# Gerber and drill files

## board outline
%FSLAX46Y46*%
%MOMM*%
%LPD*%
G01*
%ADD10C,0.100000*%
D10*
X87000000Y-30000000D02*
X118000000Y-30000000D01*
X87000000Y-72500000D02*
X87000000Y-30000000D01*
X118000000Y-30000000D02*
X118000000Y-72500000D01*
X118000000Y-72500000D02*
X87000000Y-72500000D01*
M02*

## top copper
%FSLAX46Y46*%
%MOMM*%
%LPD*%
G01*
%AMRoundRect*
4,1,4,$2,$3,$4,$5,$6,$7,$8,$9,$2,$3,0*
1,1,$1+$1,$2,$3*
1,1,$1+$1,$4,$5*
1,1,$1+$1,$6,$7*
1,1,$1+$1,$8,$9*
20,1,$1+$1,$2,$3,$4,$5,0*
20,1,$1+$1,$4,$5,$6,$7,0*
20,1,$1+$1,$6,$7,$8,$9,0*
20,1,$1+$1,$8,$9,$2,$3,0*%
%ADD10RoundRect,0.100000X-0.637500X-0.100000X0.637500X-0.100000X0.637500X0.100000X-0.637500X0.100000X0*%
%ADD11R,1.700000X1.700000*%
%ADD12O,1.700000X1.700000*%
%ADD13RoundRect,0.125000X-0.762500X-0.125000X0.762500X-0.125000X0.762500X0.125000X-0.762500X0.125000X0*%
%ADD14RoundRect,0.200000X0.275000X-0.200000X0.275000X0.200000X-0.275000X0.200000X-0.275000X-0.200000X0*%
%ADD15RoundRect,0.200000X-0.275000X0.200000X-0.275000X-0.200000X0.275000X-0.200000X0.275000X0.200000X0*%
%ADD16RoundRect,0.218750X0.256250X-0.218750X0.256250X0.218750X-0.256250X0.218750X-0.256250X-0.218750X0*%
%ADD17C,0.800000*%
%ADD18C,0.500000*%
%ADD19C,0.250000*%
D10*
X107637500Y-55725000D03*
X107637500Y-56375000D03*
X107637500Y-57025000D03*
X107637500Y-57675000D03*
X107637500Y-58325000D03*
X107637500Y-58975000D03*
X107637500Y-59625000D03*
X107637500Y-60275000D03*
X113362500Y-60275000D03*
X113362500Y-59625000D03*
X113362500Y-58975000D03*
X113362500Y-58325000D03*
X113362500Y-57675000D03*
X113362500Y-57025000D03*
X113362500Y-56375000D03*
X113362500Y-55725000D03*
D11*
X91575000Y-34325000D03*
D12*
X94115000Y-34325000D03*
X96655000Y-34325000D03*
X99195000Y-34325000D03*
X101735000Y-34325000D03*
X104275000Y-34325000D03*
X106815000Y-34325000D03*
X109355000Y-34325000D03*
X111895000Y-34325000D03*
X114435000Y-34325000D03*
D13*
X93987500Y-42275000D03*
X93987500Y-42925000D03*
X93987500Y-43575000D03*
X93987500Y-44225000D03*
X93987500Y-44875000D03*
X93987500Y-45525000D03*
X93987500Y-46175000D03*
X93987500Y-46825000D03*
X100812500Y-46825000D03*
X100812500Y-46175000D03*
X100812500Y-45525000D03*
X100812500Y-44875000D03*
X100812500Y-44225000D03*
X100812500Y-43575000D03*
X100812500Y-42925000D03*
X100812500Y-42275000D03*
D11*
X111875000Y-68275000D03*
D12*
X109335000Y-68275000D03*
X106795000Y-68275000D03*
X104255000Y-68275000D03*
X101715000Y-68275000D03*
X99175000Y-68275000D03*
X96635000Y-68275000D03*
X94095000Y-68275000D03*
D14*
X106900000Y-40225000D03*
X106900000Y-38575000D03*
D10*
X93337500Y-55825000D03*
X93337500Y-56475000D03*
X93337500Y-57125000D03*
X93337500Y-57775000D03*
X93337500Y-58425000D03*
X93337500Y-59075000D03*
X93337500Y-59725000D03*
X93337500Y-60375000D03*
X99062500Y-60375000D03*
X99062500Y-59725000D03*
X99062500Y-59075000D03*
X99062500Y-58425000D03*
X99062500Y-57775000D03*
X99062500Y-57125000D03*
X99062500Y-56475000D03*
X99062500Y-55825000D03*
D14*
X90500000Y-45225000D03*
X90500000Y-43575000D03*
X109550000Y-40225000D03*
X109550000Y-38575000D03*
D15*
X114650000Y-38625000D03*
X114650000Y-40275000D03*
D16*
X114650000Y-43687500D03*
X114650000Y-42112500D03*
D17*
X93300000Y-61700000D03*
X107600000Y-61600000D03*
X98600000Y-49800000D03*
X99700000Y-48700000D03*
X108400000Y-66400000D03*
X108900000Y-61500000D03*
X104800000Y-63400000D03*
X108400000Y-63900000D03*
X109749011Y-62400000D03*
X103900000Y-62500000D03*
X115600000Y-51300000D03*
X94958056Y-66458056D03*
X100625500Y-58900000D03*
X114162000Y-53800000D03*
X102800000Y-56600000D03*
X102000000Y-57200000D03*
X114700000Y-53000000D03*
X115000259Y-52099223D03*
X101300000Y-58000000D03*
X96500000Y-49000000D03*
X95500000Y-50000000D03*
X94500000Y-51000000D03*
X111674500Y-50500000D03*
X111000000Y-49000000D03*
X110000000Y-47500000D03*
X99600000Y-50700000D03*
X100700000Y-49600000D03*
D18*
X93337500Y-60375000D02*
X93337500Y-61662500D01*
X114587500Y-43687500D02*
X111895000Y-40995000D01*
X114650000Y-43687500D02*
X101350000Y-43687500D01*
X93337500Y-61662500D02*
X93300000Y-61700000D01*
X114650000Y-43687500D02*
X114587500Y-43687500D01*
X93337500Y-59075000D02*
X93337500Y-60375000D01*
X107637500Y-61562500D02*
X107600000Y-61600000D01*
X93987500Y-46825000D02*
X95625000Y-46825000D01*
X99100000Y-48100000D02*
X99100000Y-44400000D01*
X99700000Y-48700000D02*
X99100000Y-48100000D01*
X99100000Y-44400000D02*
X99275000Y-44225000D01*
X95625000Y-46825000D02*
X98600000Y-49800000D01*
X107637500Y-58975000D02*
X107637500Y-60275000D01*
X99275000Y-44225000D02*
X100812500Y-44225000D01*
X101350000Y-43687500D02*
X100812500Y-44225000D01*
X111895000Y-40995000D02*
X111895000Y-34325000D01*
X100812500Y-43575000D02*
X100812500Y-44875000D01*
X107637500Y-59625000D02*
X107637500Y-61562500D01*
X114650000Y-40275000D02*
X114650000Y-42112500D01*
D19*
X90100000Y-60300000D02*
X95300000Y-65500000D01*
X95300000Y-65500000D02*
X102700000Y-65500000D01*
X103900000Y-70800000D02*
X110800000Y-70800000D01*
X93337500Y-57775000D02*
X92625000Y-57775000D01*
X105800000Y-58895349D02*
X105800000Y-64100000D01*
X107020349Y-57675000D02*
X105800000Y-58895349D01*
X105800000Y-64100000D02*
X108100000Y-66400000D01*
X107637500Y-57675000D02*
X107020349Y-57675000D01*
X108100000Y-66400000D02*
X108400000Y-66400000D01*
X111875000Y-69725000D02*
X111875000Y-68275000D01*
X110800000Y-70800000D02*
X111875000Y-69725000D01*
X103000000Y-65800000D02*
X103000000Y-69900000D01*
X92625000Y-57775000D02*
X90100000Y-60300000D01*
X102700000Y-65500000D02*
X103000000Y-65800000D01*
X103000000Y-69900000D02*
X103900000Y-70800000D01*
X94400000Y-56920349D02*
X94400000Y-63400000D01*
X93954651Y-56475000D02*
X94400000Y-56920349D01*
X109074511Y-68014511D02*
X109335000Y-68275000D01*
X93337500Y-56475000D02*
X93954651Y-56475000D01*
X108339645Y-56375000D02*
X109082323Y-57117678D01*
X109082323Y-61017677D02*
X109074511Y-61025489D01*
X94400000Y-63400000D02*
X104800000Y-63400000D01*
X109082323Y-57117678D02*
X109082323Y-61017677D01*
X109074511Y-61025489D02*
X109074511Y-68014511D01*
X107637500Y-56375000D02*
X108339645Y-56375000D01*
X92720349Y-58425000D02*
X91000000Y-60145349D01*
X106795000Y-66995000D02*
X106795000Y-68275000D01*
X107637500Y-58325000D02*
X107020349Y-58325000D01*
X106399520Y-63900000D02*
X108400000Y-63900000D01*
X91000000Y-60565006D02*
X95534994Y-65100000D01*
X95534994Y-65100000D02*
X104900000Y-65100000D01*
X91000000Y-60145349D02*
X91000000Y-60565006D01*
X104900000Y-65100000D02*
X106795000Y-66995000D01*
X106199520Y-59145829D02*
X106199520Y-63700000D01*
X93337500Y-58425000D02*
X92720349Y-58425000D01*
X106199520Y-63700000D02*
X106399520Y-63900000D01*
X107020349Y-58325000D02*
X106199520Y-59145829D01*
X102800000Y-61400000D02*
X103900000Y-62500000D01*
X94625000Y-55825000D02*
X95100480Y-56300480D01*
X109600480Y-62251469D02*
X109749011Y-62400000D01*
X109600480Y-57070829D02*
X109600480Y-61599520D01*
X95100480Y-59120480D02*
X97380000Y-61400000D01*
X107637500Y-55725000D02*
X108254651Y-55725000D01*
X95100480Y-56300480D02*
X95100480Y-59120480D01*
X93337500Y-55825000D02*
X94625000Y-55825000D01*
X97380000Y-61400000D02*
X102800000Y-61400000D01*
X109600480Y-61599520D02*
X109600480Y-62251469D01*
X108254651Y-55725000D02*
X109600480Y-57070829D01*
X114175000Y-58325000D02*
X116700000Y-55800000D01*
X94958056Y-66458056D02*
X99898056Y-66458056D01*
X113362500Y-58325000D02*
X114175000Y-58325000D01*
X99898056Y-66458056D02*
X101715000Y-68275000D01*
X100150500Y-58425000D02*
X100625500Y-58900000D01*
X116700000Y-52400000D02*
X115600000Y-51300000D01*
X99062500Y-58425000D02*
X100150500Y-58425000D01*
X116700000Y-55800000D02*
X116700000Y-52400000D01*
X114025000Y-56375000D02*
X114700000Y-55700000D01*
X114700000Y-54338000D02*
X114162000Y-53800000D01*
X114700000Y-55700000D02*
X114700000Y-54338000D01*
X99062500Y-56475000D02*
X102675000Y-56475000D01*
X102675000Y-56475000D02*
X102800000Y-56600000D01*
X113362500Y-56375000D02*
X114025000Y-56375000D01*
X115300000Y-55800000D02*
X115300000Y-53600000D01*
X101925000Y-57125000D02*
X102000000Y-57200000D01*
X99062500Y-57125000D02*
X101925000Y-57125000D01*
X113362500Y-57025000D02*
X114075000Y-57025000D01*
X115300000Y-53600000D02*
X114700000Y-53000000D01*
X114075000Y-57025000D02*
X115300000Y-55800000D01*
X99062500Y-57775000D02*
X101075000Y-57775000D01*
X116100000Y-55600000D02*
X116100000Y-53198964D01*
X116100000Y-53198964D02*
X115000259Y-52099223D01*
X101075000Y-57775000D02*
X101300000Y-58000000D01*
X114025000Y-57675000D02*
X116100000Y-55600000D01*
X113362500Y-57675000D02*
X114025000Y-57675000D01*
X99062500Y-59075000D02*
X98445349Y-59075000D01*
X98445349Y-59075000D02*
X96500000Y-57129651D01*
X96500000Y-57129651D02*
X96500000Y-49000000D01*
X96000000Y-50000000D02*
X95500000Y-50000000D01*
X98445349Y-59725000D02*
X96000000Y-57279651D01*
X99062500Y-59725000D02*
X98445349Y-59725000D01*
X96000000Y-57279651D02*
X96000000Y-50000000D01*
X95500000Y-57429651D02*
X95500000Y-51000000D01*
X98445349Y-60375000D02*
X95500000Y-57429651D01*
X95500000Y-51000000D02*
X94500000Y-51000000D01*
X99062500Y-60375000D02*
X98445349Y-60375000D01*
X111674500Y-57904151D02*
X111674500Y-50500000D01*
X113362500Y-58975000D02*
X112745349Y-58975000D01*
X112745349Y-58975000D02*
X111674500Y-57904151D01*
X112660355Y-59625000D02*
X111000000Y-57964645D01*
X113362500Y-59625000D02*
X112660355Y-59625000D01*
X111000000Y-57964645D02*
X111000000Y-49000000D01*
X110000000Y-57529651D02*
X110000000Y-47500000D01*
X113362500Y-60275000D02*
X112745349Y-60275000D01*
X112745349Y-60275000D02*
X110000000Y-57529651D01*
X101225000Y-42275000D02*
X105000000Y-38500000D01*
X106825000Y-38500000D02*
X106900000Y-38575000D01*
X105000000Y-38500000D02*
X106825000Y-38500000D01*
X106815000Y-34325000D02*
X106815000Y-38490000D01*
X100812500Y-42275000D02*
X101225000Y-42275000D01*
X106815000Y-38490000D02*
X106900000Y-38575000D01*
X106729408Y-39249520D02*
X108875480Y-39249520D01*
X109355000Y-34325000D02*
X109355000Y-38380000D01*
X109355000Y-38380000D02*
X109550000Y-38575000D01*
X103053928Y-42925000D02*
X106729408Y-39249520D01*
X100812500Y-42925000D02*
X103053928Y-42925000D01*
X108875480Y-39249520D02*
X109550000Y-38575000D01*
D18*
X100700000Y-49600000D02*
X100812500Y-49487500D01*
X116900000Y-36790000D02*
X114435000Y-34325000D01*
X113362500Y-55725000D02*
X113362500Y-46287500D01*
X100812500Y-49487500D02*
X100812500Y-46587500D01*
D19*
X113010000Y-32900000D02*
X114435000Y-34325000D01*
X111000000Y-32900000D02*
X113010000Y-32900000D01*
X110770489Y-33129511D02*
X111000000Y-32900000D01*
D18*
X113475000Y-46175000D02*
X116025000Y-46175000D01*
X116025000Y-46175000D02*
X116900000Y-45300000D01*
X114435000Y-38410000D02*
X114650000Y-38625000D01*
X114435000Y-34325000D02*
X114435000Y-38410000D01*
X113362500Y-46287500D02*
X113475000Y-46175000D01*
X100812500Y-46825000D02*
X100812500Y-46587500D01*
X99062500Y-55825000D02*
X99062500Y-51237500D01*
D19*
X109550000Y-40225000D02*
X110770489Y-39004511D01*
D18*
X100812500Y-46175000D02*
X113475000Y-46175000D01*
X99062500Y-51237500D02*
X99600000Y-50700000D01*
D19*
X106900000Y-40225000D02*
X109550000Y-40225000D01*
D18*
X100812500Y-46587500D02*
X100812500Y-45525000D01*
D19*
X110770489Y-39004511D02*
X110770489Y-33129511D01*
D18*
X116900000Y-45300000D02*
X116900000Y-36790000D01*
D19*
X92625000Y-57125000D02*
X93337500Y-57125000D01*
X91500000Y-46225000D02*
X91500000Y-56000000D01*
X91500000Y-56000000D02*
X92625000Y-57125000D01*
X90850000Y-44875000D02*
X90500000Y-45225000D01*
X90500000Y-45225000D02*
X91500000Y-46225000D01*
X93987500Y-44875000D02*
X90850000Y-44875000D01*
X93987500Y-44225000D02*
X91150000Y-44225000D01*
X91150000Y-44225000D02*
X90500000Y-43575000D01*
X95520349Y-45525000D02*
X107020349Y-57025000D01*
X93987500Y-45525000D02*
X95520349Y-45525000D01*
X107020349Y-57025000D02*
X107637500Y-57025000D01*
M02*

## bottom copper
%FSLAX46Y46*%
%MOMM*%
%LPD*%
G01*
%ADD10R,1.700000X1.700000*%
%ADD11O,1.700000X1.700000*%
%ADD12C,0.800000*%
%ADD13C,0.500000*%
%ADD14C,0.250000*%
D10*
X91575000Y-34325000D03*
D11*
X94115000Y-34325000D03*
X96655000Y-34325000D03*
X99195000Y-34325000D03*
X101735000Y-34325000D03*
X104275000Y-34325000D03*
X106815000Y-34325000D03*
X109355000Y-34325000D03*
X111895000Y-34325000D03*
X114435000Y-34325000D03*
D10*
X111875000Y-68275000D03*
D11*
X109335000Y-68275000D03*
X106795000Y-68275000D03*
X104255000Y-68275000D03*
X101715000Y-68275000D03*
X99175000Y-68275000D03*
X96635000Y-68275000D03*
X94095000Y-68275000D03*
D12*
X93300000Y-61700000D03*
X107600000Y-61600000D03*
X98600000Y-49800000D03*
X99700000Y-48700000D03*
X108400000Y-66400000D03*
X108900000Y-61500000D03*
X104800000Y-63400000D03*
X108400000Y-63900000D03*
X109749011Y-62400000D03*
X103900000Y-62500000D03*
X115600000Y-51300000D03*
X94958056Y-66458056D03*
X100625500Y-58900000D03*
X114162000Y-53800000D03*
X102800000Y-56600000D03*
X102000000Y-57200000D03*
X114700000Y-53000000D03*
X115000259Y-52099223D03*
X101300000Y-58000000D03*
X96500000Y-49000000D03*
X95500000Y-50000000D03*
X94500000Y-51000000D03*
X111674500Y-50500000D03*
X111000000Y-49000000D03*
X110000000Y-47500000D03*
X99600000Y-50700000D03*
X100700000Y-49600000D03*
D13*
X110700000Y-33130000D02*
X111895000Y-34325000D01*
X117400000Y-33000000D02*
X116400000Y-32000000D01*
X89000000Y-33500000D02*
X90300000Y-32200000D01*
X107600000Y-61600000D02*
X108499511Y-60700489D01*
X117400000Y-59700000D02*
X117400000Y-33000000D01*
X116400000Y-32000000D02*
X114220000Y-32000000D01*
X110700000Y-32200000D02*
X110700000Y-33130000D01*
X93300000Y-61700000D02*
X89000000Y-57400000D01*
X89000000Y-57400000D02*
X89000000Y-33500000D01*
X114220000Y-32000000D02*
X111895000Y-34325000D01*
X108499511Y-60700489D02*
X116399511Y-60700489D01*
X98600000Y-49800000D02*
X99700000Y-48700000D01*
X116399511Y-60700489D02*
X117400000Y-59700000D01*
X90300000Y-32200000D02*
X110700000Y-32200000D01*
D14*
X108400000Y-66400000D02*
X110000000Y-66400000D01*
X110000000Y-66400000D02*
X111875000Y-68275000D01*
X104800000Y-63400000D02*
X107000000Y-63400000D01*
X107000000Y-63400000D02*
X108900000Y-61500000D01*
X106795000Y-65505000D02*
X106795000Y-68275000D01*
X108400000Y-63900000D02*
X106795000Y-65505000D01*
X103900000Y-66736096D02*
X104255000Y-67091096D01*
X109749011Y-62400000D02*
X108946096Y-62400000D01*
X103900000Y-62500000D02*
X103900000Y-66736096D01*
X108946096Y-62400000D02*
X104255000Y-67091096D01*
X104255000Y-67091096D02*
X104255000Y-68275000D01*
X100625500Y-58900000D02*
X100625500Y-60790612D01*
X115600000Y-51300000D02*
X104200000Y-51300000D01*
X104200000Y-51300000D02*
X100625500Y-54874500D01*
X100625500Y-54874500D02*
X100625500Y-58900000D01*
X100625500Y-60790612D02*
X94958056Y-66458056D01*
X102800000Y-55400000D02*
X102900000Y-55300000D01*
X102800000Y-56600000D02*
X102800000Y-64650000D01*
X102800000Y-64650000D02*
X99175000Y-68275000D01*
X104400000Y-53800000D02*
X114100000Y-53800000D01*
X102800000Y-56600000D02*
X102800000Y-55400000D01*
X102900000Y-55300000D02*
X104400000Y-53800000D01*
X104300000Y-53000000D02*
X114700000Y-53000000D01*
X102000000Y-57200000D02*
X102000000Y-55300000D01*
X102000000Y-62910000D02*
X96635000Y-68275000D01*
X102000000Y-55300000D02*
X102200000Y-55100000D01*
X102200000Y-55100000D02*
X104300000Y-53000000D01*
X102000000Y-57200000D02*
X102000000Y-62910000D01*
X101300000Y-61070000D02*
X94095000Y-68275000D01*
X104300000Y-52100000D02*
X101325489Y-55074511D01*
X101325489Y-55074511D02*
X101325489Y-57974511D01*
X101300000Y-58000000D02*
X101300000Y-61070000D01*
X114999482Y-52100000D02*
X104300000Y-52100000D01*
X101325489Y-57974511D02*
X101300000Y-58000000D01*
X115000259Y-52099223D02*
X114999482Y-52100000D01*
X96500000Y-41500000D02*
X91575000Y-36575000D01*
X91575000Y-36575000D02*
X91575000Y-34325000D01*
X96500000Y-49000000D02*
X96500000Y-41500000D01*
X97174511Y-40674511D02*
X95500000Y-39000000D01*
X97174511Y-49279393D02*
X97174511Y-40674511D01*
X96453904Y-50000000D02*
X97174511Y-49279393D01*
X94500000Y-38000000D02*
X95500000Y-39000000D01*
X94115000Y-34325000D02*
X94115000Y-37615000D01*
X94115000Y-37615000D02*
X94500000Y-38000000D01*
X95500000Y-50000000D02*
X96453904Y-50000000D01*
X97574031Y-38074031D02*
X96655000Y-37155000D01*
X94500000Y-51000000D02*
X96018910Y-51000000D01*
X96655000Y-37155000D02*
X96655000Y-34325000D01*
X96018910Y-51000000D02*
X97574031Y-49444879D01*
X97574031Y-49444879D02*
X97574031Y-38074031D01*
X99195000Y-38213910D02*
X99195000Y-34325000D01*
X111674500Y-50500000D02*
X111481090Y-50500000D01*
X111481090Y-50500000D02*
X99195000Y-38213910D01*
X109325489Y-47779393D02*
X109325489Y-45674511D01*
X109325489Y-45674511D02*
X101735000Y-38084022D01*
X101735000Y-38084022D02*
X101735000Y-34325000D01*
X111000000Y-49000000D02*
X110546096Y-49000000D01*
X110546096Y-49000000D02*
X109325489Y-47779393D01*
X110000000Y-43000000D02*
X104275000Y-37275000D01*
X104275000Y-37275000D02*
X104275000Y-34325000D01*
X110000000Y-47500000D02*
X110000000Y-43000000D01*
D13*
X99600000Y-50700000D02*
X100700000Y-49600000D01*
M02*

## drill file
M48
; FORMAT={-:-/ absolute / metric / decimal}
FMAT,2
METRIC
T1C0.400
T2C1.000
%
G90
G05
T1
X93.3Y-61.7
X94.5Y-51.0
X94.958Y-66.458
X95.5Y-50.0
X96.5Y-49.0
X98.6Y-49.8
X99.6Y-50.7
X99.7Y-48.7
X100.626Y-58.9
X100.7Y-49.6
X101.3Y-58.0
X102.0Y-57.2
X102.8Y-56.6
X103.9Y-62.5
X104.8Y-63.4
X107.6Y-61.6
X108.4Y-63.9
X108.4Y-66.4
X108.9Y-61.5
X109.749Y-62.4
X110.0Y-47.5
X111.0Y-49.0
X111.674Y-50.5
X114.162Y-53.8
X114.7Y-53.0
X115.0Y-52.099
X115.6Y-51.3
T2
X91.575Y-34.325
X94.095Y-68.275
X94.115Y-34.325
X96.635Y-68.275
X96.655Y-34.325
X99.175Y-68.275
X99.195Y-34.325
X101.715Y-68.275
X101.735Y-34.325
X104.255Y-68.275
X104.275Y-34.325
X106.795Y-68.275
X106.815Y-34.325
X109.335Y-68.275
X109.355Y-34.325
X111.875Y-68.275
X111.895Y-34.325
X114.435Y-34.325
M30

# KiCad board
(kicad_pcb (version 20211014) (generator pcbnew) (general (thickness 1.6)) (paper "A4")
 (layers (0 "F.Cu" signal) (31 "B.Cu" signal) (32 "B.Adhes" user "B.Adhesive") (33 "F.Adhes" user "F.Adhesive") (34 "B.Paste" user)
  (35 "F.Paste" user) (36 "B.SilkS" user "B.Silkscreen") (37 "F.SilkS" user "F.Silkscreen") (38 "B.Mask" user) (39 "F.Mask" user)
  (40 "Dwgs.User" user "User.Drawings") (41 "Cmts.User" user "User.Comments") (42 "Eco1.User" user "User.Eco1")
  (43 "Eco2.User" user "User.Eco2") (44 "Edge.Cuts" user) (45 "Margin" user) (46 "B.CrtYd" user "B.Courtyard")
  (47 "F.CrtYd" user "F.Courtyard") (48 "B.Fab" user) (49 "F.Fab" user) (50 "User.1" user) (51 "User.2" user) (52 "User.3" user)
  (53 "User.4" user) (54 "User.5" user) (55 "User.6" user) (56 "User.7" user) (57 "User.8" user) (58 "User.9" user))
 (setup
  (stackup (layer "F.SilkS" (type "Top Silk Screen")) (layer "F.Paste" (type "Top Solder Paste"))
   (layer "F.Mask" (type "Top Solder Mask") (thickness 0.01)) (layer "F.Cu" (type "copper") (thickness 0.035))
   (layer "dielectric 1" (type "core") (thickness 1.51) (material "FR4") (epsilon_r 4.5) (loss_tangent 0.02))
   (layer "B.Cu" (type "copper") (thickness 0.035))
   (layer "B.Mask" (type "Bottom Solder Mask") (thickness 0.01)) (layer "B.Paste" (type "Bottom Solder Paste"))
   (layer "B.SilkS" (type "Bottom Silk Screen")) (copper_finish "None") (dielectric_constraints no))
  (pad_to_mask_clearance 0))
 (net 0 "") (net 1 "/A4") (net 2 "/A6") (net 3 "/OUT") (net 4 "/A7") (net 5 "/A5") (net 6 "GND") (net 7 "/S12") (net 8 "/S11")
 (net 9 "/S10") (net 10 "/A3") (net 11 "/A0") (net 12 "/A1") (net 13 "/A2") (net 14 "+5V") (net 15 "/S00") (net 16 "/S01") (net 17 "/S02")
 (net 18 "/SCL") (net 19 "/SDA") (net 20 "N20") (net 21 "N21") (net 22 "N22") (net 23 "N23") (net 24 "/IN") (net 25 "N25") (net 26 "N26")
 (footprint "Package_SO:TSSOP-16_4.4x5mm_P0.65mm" (layer "F.Cu") (at 110.5 58)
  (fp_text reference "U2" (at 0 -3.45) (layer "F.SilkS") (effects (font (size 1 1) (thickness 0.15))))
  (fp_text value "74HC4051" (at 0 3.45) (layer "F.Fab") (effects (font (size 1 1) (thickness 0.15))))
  (pad "1" smd roundrect locked (at -2.8625 -2.275) (size 1.475 0.4) (layers "F.Cu" "F.Paste" "F.Mask") (roundrect_rratio 0.25)
   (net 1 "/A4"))
  (pad "2" smd roundrect locked (at -2.8625 -1.625) (size 1.475 0.4) (layers "F.Cu" "F.Paste" "F.Mask") (roundrect_rratio 0.25)
   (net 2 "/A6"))
  (pad "3" smd roundrect locked (at -2.8625 -0.975) (size 1.475 0.4) (layers "F.Cu" "F.Paste" "F.Mask") (roundrect_rratio 0.25)
   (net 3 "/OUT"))
  (pad "4" smd roundrect locked (at -2.8625 -0.325) (size 1.475 0.4) (layers "F.Cu" "F.Paste" "F.Mask") (roundrect_rratio 0.25)
   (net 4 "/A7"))
  (pad "5" smd roundrect locked (at -2.8625 0.325) (size 1.475 0.4) (layers "F.Cu" "F.Paste" "F.Mask") (roundrect_rratio 0.25) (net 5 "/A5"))
  (pad "6" smd roundrect locked (at -2.8625 0.975) (size 1.475 0.4) (layers "F.Cu" "F.Paste" "F.Mask") (roundrect_rratio 0.25) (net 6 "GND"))
  (pad "7" smd roundrect locked (at -2.8625 1.625) (size 1.475 0.4) (layers "F.Cu" "F.Paste" "F.Mask") (roundrect_rratio 0.25) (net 6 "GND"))
  (pad "8" smd roundrect locked (at -2.8625 2.275) (size 1.475 0.4) (layers "F.Cu" "F.Paste" "F.Mask") (roundrect_rratio 0.25) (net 6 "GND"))
  (pad "9" smd roundrect locked (at 2.8625 2.275) (size 1.475 0.4) (layers "F.Cu" "F.Paste" "F.Mask") (roundrect_rratio 0.25) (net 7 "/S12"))
  (pad "10" smd roundrect locked (at 2.8625 1.625) (size 1.475 0.4) (layers "F.Cu" "F.Paste" "F.Mask") (roundrect_rratio 0.25)
   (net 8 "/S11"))
  (pad "11" smd roundrect locked (at 2.8625 0.975) (size 1.475 0.4) (layers "F.Cu" "F.Paste" "F.Mask") (roundrect_rratio 0.25)
   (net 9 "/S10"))
  (pad "12" smd roundrect locked (at 2.8625 0.325) (size 1.475 0.4) (layers "F.Cu" "F.Paste" "F.Mask") (roundrect_rratio 0.25)
   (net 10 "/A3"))
  (pad "13" smd roundrect locked (at 2.8625 -0.325) (size 1.475 0.4) (layers "F.Cu" "F.Paste" "F.Mask") (roundrect_rratio 0.25)
   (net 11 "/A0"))
  (pad "14" smd roundrect locked (at 2.8625 -0.975) (size 1.475 0.4) (layers "F.Cu" "F.Paste" "F.Mask") (roundrect_rratio 0.25)
   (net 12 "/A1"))
  (pad "15" smd roundrect locked (at 2.8625 -1.625) (size 1.475 0.4) (layers "F.Cu" "F.Paste" "F.Mask") (roundrect_rratio 0.25)
   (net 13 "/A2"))
  (pad "16" smd roundrect locked (at 2.8625 -2.275) (size 1.475 0.4) (layers "F.Cu" "F.Paste" "F.Mask") (roundrect_rratio 0.25)
   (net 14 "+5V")))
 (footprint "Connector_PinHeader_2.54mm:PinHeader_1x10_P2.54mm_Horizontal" (layer "F.Cu") (at 91.575 34.325 90)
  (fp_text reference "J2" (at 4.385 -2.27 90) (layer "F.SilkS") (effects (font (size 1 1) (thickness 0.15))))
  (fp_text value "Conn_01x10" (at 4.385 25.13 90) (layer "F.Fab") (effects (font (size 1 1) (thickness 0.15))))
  (pad "1" thru_hole rect locked (at 0 0 90) (size 1.7 1.7) (drill 1) (layers *.Cu *.Mask) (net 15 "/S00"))
  (pad "2" thru_hole oval locked (at 0 2.54 90) (size 1.7 1.7) (drill 1) (layers *.Cu *.Mask) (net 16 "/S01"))
  (pad "3" thru_hole oval locked (at 0 5.08 90) (size 1.7 1.7) (drill 1) (layers *.Cu *.Mask) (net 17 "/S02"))
  (pad "4" thru_hole oval locked (at 0 7.62 90) (size 1.7 1.7) (drill 1) (layers *.Cu *.Mask) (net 9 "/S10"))
  (pad "5" thru_hole oval locked (at 0 10.16 90) (size 1.7 1.7) (drill 1) (layers *.Cu *.Mask) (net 8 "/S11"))
  (pad "6" thru_hole oval locked (at 0 12.7 90) (size 1.7 1.7) (drill 1) (layers *.Cu *.Mask) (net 7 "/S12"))
  (pad "7" thru_hole oval locked (at 0 15.24 90) (size 1.7 1.7) (drill 1) (layers *.Cu *.Mask) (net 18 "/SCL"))
  (pad "8" thru_hole oval locked (at 0 17.78 90) (size 1.7 1.7) (drill 1) (layers *.Cu *.Mask) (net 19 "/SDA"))
  (pad "9" thru_hole oval locked (at 0 20.32 90) (size 1.7 1.7) (drill 1) (layers *.Cu *.Mask) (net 6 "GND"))
  (pad "10" thru_hole oval locked (at 0 22.86 90) (size 1.7 1.7) (drill 1) (layers *.Cu *.Mask) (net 14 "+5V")))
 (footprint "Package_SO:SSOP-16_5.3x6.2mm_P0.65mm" (layer "F.Cu") (at 97.4 44.55)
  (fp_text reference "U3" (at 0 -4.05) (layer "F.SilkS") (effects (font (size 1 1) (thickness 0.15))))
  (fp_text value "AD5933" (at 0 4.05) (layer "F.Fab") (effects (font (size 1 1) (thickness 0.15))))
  (pad "1" smd roundrect locked (at -3.4125 -2.275) (size 1.775 0.5) (layers "F.Cu" "F.Paste" "F.Mask") (roundrect_rratio 0.25)
   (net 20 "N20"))
  (pad "2" smd roundrect locked (at -3.4125 -1.625) (size 1.775 0.5) (layers "F.Cu" "F.Paste" "F.Mask") (roundrect_rratio 0.25)
   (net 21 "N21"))
  (pad "3" smd roundrect locked (at -3.4125 -0.975) (size 1.775 0.5) (layers "F.Cu" "F.Paste" "F.Mask") (roundrect_rratio 0.25)
   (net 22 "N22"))
  (pad "4" smd roundrect locked (at -3.4125 -0.325) (size 1.775 0.5) (layers "F.Cu" "F.Paste" "F.Mask") (roundrect_rratio 0.25)
   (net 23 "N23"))
  (pad "5" smd roundrect locked (at -3.4125 0.325) (size 1.775 0.5) (layers "F.Cu" "F.Paste" "F.Mask") (roundrect_rratio 0.25)
   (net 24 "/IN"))
  (pad "6" smd roundrect locked (at -3.4125 0.975) (size 1.775 0.5) (layers "F.Cu" "F.Paste" "F.Mask") (roundrect_rratio 0.25)
   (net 3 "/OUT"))
  (pad "7" smd roundrect locked (at -3.4125 1.625) (size 1.775 0.5) (layers "F.Cu" "F.Paste" "F.Mask") (roundrect_rratio 0.25)
   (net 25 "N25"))
  (pad "8" smd roundrect locked (at -3.4125 2.275) (size 1.775 0.5) (layers "F.Cu" "F.Paste" "F.Mask") (roundrect_rratio 0.25) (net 6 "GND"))
  (pad "9" smd roundrect locked (at 3.4125 2.275) (size 1.775 0.5) (layers "F.Cu" "F.Paste" "F.Mask") (roundrect_rratio 0.25) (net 14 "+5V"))
  (pad "10" smd roundrect locked (at 3.4125 1.625) (size 1.775 0.5) (layers "F.Cu" "F.Paste" "F.Mask") (roundrect_rratio 0.25)
   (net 14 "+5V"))
  (pad "11" smd roundrect locked (at 3.4125 0.975) (size 1.775 0.5) (layers "F.Cu" "F.Paste" "F.Mask") (roundrect_rratio 0.25)
   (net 14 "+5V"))
  (pad "12" smd roundrect locked (at 3.4125 0.325) (size 1.775 0.5) (layers "F.Cu" "F.Paste" "F.Mask") (roundrect_rratio 0.25) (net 6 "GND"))
  (pad "13" smd roundrect locked (at 3.4125 -0.325) (size 1.775 0.5) (layers "F.Cu" "F.Paste" "F.Mask") (roundrect_rratio 0.25)
   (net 6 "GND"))
  (pad "14" smd roundrect locked (at 3.4125 -0.975) (size 1.775 0.5) (layers "F.Cu" "F.Paste" "F.Mask") (roundrect_rratio 0.25)
   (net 6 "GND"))
  (pad "15" smd roundrect locked (at 3.4125 -1.625) (size 1.775 0.5) (layers "F.Cu" "F.Paste" "F.Mask") (roundrect_rratio 0.25)
   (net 19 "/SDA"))
  (pad "16" smd roundrect locked (at 3.4125 -2.275) (size 1.775 0.5) (layers "F.Cu" "F.Paste" "F.Mask") (roundrect_rratio 0.25)
   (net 18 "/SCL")))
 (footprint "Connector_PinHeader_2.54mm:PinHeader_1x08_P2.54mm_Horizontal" (layer "F.Cu") (at 111.875 68.275 -90)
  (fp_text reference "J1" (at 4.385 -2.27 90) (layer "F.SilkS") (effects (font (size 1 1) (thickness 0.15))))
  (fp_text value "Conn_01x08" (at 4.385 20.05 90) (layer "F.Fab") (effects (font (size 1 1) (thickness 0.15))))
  (pad "1" thru_hole rect locked (at 0 0 270) (size 1.7 1.7) (drill 1) (layers *.Cu *.Mask) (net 4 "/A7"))
  (pad "2" thru_hole oval locked (at 0 2.54 270) (size 1.7 1.7) (drill 1) (layers *.Cu *.Mask) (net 2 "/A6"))
  (pad "3" thru_hole oval locked (at 0 5.08 270) (size 1.7 1.7) (drill 1) (layers *.Cu *.Mask) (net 5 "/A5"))
  (pad "4" thru_hole oval locked (at 0 7.62 270) (size 1.7 1.7) (drill 1) (layers *.Cu *.Mask) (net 1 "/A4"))
  (pad "5" thru_hole oval locked (at 0 10.16 270) (size 1.7 1.7) (drill 1) (layers *.Cu *.Mask) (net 10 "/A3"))
  (pad "6" thru_hole oval locked (at 0 12.7 270) (size 1.7 1.7) (drill 1) (layers *.Cu *.Mask) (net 13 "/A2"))
  (pad "7" thru_hole oval locked (at 0 15.24 270) (size 1.7 1.7) (drill 1) (layers *.Cu *.Mask) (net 12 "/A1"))
  (pad "8" thru_hole oval locked (at 0 17.78 270) (size 1.7 1.7) (drill 1) (layers *.Cu *.Mask) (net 11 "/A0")))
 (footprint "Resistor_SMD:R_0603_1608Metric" (layer "F.Cu") (at 106.9 39.4 90)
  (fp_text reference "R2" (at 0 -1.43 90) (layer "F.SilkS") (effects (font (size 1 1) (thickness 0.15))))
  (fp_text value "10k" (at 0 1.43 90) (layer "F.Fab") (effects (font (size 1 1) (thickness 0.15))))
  (pad "1" smd roundrect locked (at -0.825 0 90) (size 0.8 0.95) (layers "F.Cu" "F.Paste" "F.Mask") (roundrect_rratio 0.25) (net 14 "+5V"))
  (pad "2" smd roundrect locked (at 0.825 0 90) (size 0.8 0.95) (layers "F.Cu" "F.Paste" "F.Mask") (roundrect_rratio 0.25) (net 18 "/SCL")))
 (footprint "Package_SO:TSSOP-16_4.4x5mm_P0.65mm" (layer "F.Cu") (at 96.2 58.1)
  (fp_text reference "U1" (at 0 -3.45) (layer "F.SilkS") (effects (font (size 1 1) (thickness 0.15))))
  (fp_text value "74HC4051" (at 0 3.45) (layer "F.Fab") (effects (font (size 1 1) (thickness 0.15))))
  (pad "1" smd roundrect locked (at -2.8625 -2.275) (size 1.475 0.4) (layers "F.Cu" "F.Paste" "F.Mask") (roundrect_rratio 0.25)
   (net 1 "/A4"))
  (pad "2" smd roundrect locked (at -2.8625 -1.625) (size 1.475 0.4) (layers "F.Cu" "F.Paste" "F.Mask") (roundrect_rratio 0.25)
   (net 2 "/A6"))
  (pad "3" smd roundrect locked (at -2.8625 -0.975) (size 1.475 0.4) (layers "F.Cu" "F.Paste" "F.Mask") (roundrect_rratio 0.25)
   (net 24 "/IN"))
  (pad "4" smd roundrect locked (at -2.8625 -0.325) (size 1.475 0.4) (layers "F.Cu" "F.Paste" "F.Mask") (roundrect_rratio 0.25)
   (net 4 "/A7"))
  (pad "5" smd roundrect locked (at -2.8625 0.325) (size 1.475 0.4) (layers "F.Cu" "F.Paste" "F.Mask") (roundrect_rratio 0.25) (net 5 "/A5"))
  (pad "6" smd roundrect locked (at -2.8625 0.975) (size 1.475 0.4) (layers "F.Cu" "F.Paste" "F.Mask") (roundrect_rratio 0.25) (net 6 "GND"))
  (pad "7" smd roundrect locked (at -2.8625 1.625) (size 1.475 0.4) (layers "F.Cu" "F.Paste" "F.Mask") (roundrect_rratio 0.25) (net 6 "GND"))
  (pad "8" smd roundrect locked (at -2.8625 2.275) (size 1.475 0.4) (layers "F.Cu" "F.Paste" "F.Mask") (roundrect_rratio 0.25) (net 6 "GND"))
  (pad "9" smd roundrect locked (at 2.8625 2.275) (size 1.475 0.4) (layers "F.Cu" "F.Paste" "F.Mask") (roundrect_rratio 0.25)
   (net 17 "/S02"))
  (pad "10" smd roundrect locked (at 2.8625 1.625) (size 1.475 0.4) (layers "F.Cu" "F.Paste" "F.Mask") (roundrect_rratio 0.25)
   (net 16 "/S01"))
  (pad "11" smd roundrect locked (at 2.8625 0.975) (size 1.475 0.4) (layers "F.Cu" "F.Paste" "F.Mask") (roundrect_rratio 0.25)
   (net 15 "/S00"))
  (pad "12" smd roundrect locked (at 2.8625 0.325) (size 1.475 0.4) (layers "F.Cu" "F.Paste" "F.Mask") (roundrect_rratio 0.25)
   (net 10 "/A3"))
  (pad "13" smd roundrect locked (at 2.8625 -0.325) (size 1.475 0.4) (layers "F.Cu" "F.Paste" "F.Mask") (roundrect_rratio 0.25)
   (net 11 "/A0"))
  (pad "14" smd roundrect locked (at 2.8625 -0.975) (size 1.475 0.4) (layers "F.Cu" "F.Paste" "F.Mask") (roundrect_rratio 0.25)
   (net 12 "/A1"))
  (pad "15" smd roundrect locked (at 2.8625 -1.625) (size 1.475 0.4) (layers "F.Cu" "F.Paste" "F.Mask") (roundrect_rratio 0.25)
   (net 13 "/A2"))
  (pad "16" smd roundrect locked (at 2.8625 -2.275) (size 1.475 0.4) (layers "F.Cu" "F.Paste" "F.Mask") (roundrect_rratio 0.25)
   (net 14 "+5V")))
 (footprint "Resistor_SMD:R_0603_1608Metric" (layer "F.Cu") (at 90.5 44.4 90)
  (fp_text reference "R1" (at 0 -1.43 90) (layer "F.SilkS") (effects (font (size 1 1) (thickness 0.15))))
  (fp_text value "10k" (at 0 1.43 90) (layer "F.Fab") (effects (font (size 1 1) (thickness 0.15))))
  (pad "1" smd roundrect locked (at -0.825 0 90) (size 0.8 0.95) (layers "F.Cu" "F.Paste" "F.Mask") (roundrect_rratio 0.25) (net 24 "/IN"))
  (pad "2" smd roundrect locked (at 0.825 0 90) (size 0.8 0.95) (layers "F.Cu" "F.Paste" "F.Mask") (roundrect_rratio 0.25) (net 23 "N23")))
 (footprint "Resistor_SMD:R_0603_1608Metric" (layer "F.Cu") (at 109.55 39.4 90)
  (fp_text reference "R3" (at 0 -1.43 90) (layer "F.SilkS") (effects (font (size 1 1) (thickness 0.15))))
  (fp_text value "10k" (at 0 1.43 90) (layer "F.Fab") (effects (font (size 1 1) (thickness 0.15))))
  (pad "1" smd roundrect locked (at -0.825 0 90) (size 0.8 0.95) (layers "F.Cu" "F.Paste" "F.Mask") (roundrect_rratio 0.25) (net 14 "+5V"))
  (pad "2" smd roundrect locked (at 0.825 0 90) (size 0.8 0.95) (layers "F.Cu" "F.Paste" "F.Mask") (roundrect_rratio 0.25) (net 19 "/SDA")))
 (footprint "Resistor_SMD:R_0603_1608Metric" (layer "F.Cu") (at 114.65 39.45 -90)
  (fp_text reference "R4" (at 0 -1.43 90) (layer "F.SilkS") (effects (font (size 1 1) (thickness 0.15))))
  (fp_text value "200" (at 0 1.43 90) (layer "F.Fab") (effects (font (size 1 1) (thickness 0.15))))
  (pad "1" smd roundrect locked (at -0.825 0 270) (size 0.8 0.95) (layers "F.Cu" "F.Paste" "F.Mask") (roundrect_rratio 0.25) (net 14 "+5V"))
  (pad "2" smd roundrect locked (at 0.825 0 270) (size 0.8 0.95) (layers "F.Cu" "F.Paste" "F.Mask") (roundrect_rratio 0.25) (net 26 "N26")))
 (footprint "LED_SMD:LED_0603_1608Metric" (layer "F.Cu") (at 114.65 42.9 90)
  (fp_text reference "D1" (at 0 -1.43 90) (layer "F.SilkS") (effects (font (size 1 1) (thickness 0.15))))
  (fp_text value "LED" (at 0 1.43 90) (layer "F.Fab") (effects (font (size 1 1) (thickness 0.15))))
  (pad "1" smd roundrect locked (at -0.7875 0 90) (size 0.875 0.95) (layers "F.Cu" "F.Paste" "F.Mask") (roundrect_rratio 0.25) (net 6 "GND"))
  (pad "2" smd roundrect locked (at 0.7875 0 90) (size 0.875 0.95) (layers "F.Cu" "F.Paste" "F.Mask") (roundrect_rratio 0.25) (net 26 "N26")))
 (gr_line (start 87 30) (end 118 30) (layer "Edge.Cuts") (width 0.1))
 (gr_line (start 87 72.5) (end 87 30) (layer "Edge.Cuts") (width 0.1))
 (gr_line (start 118 30) (end 118 72.5) (layer "Edge.Cuts") (width 0.1))
 (gr_line (start 118 72.5) (end 87 72.5) (layer "Edge.Cuts") (width 0.1))
 (segment (start 93.3375 60.375) (end 93.3375 61.6625) (width 0.5) (layer "F.Cu") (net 6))
 (segment (start 114.5875 43.6875) (end 111.895 40.995) (width 0.5) (layer "F.Cu") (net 6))
 (segment (start 114.65 43.6875) (end 101.35 43.6875) (width 0.5) (layer "F.Cu") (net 6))
 (segment (start 93.3375 61.6625) (end 93.3 61.7) (width 0.5) (layer "F.Cu") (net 6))
 (segment (start 114.65 43.6875) (end 114.5875 43.6875) (width 0.5) (layer "F.Cu") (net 6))
 (segment (start 93.3375 59.075) (end 93.3375 60.375) (width 0.5) (layer "F.Cu") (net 6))
 (segment (start 107.6375 61.5625) (end 107.6 61.6) (width 0.5) (layer "F.Cu") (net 6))
 (segment (start 93.9875 46.825) (end 95.625 46.825) (width 0.5) (layer "F.Cu") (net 6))
 (segment (start 99.1 48.1) (end 99.1 44.4) (width 0.5) (layer "F.Cu") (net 6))
 (segment (start 99.7 48.7) (end 99.1 48.1) (width 0.5) (layer "F.Cu") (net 6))
 (segment (start 99.1 44.4) (end 99.275 44.225) (width 0.5) (layer "F.Cu") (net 6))
 (segment (start 95.625 46.825) (end 98.6 49.8) (width 0.5) (layer "F.Cu") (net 6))
 (segment (start 107.6375 58.975) (end 107.6375 60.275) (width 0.5) (layer "F.Cu") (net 6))
 (segment (start 99.275 44.225) (end 100.8125 44.225) (width 0.5) (layer "F.Cu") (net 6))
 (segment (start 101.35 43.6875) (end 100.8125 44.225) (width 0.5) (layer "F.Cu") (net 6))
 (segment (start 111.895 40.995) (end 111.895 34.325) (width 0.5) (layer "F.Cu") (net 6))
 (segment (start 100.8125 43.575) (end 100.8125 44.875) (width 0.5) (layer "F.Cu") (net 6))
 (segment (start 107.6375 59.625) (end 107.6375 61.5625) (width 0.5) (layer "F.Cu") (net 6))
 (via (at 93.3 61.7) (size 0.8) (drill 0.4) (layers "F.Cu" "B.Cu") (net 6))
 (via (at 107.6 61.6) (size 0.8) (drill 0.4) (layers "F.Cu" "B.Cu") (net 6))
 (via (at 98.6 49.8) (size 0.8) (drill 0.4) (layers "F.Cu" "B.Cu") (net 6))
 (via (at 99.7 48.7) (size 0.8) (drill 0.4) (layers "F.Cu" "B.Cu") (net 6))
 (segment (start 110.7 33.13) (end 111.895 34.325) (width 0.5) (layer "B.Cu") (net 6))
 (segment (start 117.4 33) (end 116.4 32) (width 0.5) (layer "B.Cu") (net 6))
 (segment (start 89 33.5) (end 90.3 32.2) (width 0.5) (layer "B.Cu") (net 6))
 (segment (start 107.6 61.6) (end 108.499511 60.700489) (width 0.5) (layer "B.Cu") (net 6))
 (segment (start 117.4 59.7) (end 117.4 33) (width 0.5) (layer "B.Cu") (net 6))
 (segment (start 116.4 32) (end 114.22 32) (width 0.5) (layer "B.Cu") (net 6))
 (segment (start 110.7 32.2) (end 110.7 33.13) (width 0.5) (layer "B.Cu") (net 6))
 (segment (start 93.3 61.7) (end 89 57.4) (width 0.5) (layer "B.Cu") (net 6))
 (segment (start 89 57.4) (end 89 33.5) (width 0.5) (layer "B.Cu") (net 6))
 (segment (start 114.22 32) (end 111.895 34.325) (width 0.5) (layer "B.Cu") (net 6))
 (segment (start 108.499511 60.700489) (end 116.399511 60.700489) (width 0.5) (layer "B.Cu") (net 6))
 (segment (start 98.6 49.8) (end 99.7 48.7) (width 0.5) (layer "B.Cu") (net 6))
 (segment (start 116.399511 60.700489) (end 117.4 59.7) (width 0.5) (layer "B.Cu") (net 6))
 (segment (start 90.3 32.2) (end 110.7 32.2) (width 0.5) (layer "B.Cu") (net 6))
 (segment (start 114.65 40.275) (end 114.65 42.1125) (width 0.5) (layer "F.Cu") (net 26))
 (segment (start 90.1 60.3) (end 95.3 65.5) (width 0.25) (layer "F.Cu") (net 4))
 (segment (start 95.3 65.5) (end 102.7 65.5) (width 0.25) (layer "F.Cu") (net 4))
 (segment (start 103.9 70.8) (end 110.8 70.8) (width 0.25) (layer "F.Cu") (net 4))
 (segment (start 93.3375 57.775) (end 92.625 57.775) (width 0.25) (layer "F.Cu") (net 4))
 (segment (start 105.8 58.895349) (end 105.8 64.1) (width 0.25) (layer "F.Cu") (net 4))
 (segment (start 107.020349 57.675) (end 105.8 58.895349) (width 0.25) (layer "F.Cu") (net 4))
 (segment (start 105.8 64.1) (end 108.1 66.4) (width 0.25) (layer "F.Cu") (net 4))
 (segment (start 107.6375 57.675) (end 107.020349 57.675) (width 0.25) (layer "F.Cu") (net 4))
 (segment (start 108.1 66.4) (end 108.4 66.4) (width 0.25) (layer "F.Cu") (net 4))
 (segment (start 111.875 69.725) (end 111.875 68.275) (width 0.25) (layer "F.Cu") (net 4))
 (segment (start 110.8 70.8) (end 111.875 69.725) (width 0.25) (layer "F.Cu") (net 4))
 (segment (start 103 65.8) (end 103 69.9) (width 0.25) (layer "F.Cu") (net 4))
 (segment (start 92.625 57.775) (end 90.1 60.3) (width 0.25) (layer "F.Cu") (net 4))
 (segment (start 102.7 65.5) (end 103 65.8) (width 0.25) (layer "F.Cu") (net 4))
 (segment (start 103 69.9) (end 103.9 70.8) (width 0.25) (layer "F.Cu") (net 4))
 (via (at 108.4 66.4) (size 0.8) (drill 0.4) (layers "F.Cu" "B.Cu") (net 4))
 (segment (start 108.4 66.4) (end 110 66.4) (width 0.25) (layer "B.Cu") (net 4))
 (segment (start 110 66.4) (end 111.875 68.275) (width 0.25) (layer "B.Cu") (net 4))
 (segment (start 94.4 56.920349) (end 94.4 63.4) (width 0.25) (layer "F.Cu") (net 2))
 (segment (start 93.954651 56.475) (end 94.4 56.920349) (width 0.25) (layer "F.Cu") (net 2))
 (segment (start 109.074511 68.014511) (end 109.335 68.275) (width 0.25) (layer "F.Cu") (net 2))
 (segment (start 93.3375 56.475) (end 93.954651 56.475) (width 0.25) (layer "F.Cu") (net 2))
 (segment (start 108.339645 56.375) (end 109.082323 57.117678) (width 0.25) (layer "F.Cu") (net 2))
 (segment (start 109.082323 61.017677) (end 109.074511 61.025489) (width 0.25) (layer "F.Cu") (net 2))
 (segment (start 94.4 63.4) (end 104.8 63.4) (width 0.25) (layer "F.Cu") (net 2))
 (segment (start 109.082323 57.117678) (end 109.082323 61.017677) (width 0.25) (layer "F.Cu") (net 2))
 (segment (start 109.074511 61.025489) (end 109.074511 68.014511) (width 0.25) (layer "F.Cu") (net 2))
 (segment (start 107.6375 56.375) (end 108.339645 56.375) (width 0.25) (layer "F.Cu") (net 2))
 (via (at 108.9 61.5) (size 0.8) (drill 0.4) (layers "F.Cu" "B.Cu") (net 2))
 (via (at 104.8 63.4) (size 0.8) (drill 0.4) (layers "F.Cu" "B.Cu") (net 2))
 (segment (start 104.8 63.4) (end 107 63.4) (width 0.25) (layer "B.Cu") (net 2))
 (segment (start 107 63.4) (end 108.9 61.5) (width 0.25) (layer "B.Cu") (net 2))
 (segment (start 92.720349 58.425) (end 91 60.145349) (width 0.25) (layer "F.Cu") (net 5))
 (segment (start 106.795 66.995) (end 106.795 68.275) (width 0.25) (layer "F.Cu") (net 5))
 (segment (start 107.6375 58.325) (end 107.020349 58.325) (width 0.25) (layer "F.Cu") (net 5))
 (segment (start 106.39952 63.9) (end 108.4 63.9) (width 0.25) (layer "F.Cu") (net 5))
 (segment (start 91 60.565006) (end 95.534994 65.1) (width 0.25) (layer "F.Cu") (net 5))
 (segment (start 95.534994 65.1) (end 104.9 65.1) (width 0.25) (layer "F.Cu") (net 5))
 (segment (start 91 60.145349) (end 91 60.565006) (width 0.25) (layer "F.Cu") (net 5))
 (segment (start 104.9 65.1) (end 106.795 66.995) (width 0.25) (layer "F.Cu") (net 5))
 (segment (start 106.19952 59.145829) (end 106.19952 63.7) (width 0.25) (layer "F.Cu") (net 5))
 (segment (start 93.3375 58.425) (end 92.720349 58.425) (width 0.25) (layer "F.Cu") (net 5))
 (segment (start 106.19952 63.7) (end 106.39952 63.9) (width 0.25) (layer "F.Cu") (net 5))
 (segment (start 107.020349 58.325) (end 106.19952 59.145829) (width 0.25) (layer "F.Cu") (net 5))
 (via (at 108.4 63.9) (size 0.8) (drill 0.4) (layers "F.Cu" "B.Cu") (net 5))
 (segment (start 106.795 65.505) (end 106.795 68.275) (width 0.25) (layer "B.Cu") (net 5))
 (segment (start 108.4 63.9) (end 106.795 65.505) (width 0.25) (layer "B.Cu") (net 5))
 (segment (start 102.8 61.4) (end 103.9 62.5) (width 0.25) (layer "F.Cu") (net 1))
 (segment (start 94.625 55.825) (end 95.10048 56.30048) (width 0.25) (layer "F.Cu") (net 1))
 (segment (start 109.60048 62.251469) (end 109.749011 62.4) (width 0.25) (layer "F.Cu") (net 1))
 (segment (start 109.60048 57.070829) (end 109.60048 61.59952) (width 0.25) (layer "F.Cu") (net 1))
 (segment (start 95.10048 59.12048) (end 97.38 61.4) (width 0.25) (layer "F.Cu") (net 1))
 (segment (start 107.6375 55.725) (end 108.254651 55.725) (width 0.25) (layer "F.Cu") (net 1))
 (segment (start 95.10048 56.30048) (end 95.10048 59.12048) (width 0.25) (layer "F.Cu") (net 1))
 (segment (start 93.3375 55.825) (end 94.625 55.825) (width 0.25) (layer "F.Cu") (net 1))
 (segment (start 97.38 61.4) (end 102.8 61.4) (width 0.25) (layer "F.Cu") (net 1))
 (segment (start 109.60048 61.59952) (end 109.60048 62.251469) (width 0.25) (layer "F.Cu") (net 1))
 (segment (start 108.254651 55.725) (end 109.60048 57.070829) (width 0.25) (layer "F.Cu") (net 1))
 (via (at 109.749011 62.4) (size 0.8) (drill 0.4) (layers "F.Cu" "B.Cu") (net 1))
 (via (at 103.9 62.5) (size 0.8) (drill 0.4) (layers "F.Cu" "B.Cu") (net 1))
 (segment (start 103.9 66.736096) (end 104.255 67.091096) (width 0.25) (layer "B.Cu") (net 1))
 (segment (start 109.749011 62.4) (end 108.946096 62.4) (width 0.25) (layer "B.Cu") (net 1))
 (segment (start 103.9 62.5) (end 103.9 66.736096) (width 0.25) (layer "B.Cu") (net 1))
 (segment (start 108.946096 62.4) (end 104.255 67.091096) (width 0.25) (layer "B.Cu") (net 1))
 (segment (start 104.255 67.091096) (end 104.255 68.275) (width 0.25) (layer "B.Cu") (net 1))
 (segment (start 114.175 58.325) (end 116.7 55.8) (width 0.25) (layer "F.Cu") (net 10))
 (segment (start 94.958056 66.458056) (end 99.898056 66.458056) (width 0.25) (layer "F.Cu") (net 10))
 (segment (start 113.3625 58.325) (end 114.175 58.325) (width 0.25) (layer "F.Cu") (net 10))
 (segment (start 99.898056 66.458056) (end 101.715 68.275) (width 0.25) (layer "F.Cu") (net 10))
 (segment (start 100.1505 58.425) (end 100.6255 58.9) (width 0.25) (layer "F.Cu") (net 10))
 (segment (start 116.7 52.4) (end 115.6 51.3) (width 0.25) (layer "F.Cu") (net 10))
 (segment (start 99.0625 58.425) (end 100.1505 58.425) (width 0.25) (layer "F.Cu") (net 10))
 (segment (start 116.7 55.8) (end 116.7 52.4) (width 0.25) (layer "F.Cu") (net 10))
 (via (at 115.6 51.3) (size 0.8) (drill 0.4) (layers "F.Cu" "B.Cu") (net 10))
 (via (at 94.958056 66.458056) (size 0.8) (drill 0.4) (layers "F.Cu" "B.Cu") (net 10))
 (via (at 100.6255 58.9) (size 0.8) (drill 0.4) (layers "F.Cu" "B.Cu") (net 10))
 (segment (start 100.6255 58.9) (end 100.6255 60.790612) (width 0.25) (layer "B.Cu") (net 10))
 (segment (start 115.6 51.3) (end 104.2 51.3) (width 0.25) (layer "B.Cu") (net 10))
 (segment (start 104.2 51.3) (end 100.6255 54.8745) (width 0.25) (layer "B.Cu") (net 10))
 (segment (start 100.6255 54.8745) (end 100.6255 58.9) (width 0.25) (layer "B.Cu") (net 10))
 (segment (start 100.6255 60.790612) (end 94.958056 66.458056) (width 0.25) (layer "B.Cu") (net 10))
 (segment (start 114.025 56.375) (end 114.7 55.7) (width 0.25) (layer "F.Cu") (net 13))
 (segment (start 114.7 54.338) (end 114.162 53.8) (width 0.25) (layer "F.Cu") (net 13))
 (segment (start 114.7 55.7) (end 114.7 54.338) (width 0.25) (layer "F.Cu") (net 13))
 (segment (start 99.0625 56.475) (end 102.675 56.475) (width 0.25) (layer "F.Cu") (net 13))
 (segment (start 102.675 56.475) (end 102.8 56.6) (width 0.25) (layer "F.Cu") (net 13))
 (segment (start 113.3625 56.375) (end 114.025 56.375) (width 0.25) (layer "F.Cu") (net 13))
 (via (at 114.162 53.8) (size 0.8) (drill 0.4) (layers "F.Cu" "B.Cu") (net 13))
 (via (at 102.8 56.6) (size 0.8) (drill 0.4) (layers "F.Cu" "B.Cu") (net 13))
 (segment (start 102.8 55.4) (end 102.9 55.3) (width 0.25) (layer "B.Cu") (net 13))
 (segment (start 102.8 56.6) (end 102.8 64.65) (width 0.25) (layer "B.Cu") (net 13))
 (segment (start 102.8 64.65) (end 99.175 68.275) (width 0.25) (layer "B.Cu") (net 13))
 (segment (start 104.4 53.8) (end 114.1 53.8) (width 0.25) (layer "B.Cu") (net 13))
 (segment (start 102.8 56.6) (end 102.8 55.4) (width 0.25) (layer "B.Cu") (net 13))
 (segment (start 102.9 55.3) (end 104.4 53.8) (width 0.25) (layer "B.Cu") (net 13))
 (segment (start 115.3 55.8) (end 115.3 53.6) (width 0.25) (layer "F.Cu") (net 12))
 (segment (start 101.925 57.125) (end 102 57.2) (width 0.25) (layer "F.Cu") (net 12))
 (segment (start 99.0625 57.125) (end 101.925 57.125) (width 0.25) (layer "F.Cu") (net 12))
 (segment (start 113.3625 57.025) (end 114.075 57.025) (width 0.25) (layer "F.Cu") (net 12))
 (segment (start 115.3 53.6) (end 114.7 53) (width 0.25) (layer "F.Cu") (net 12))
 (segment (start 114.075 57.025) (end 115.3 55.8) (width 0.25) (layer "F.Cu") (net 12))
 (via (at 102 57.2) (size 0.8) (drill 0.4) (layers "F.Cu" "B.Cu") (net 12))
 (via (at 114.7 53) (size 0.8) (drill 0.4) (layers "F.Cu" "B.Cu") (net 12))
 (segment (start 104.3 53) (end 114.7 53) (width 0.25) (layer "B.Cu") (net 12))
 (segment (start 102 57.2) (end 102 55.3) (width 0.25) (layer "B.Cu") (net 12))
 (segment (start 102 62.91) (end 96.635 68.275) (width 0.25) (layer "B.Cu") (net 12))
 (segment (start 102 55.3) (end 102.2 55.1) (width 0.25) (layer "B.Cu") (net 12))
 (segment (start 102.2 55.1) (end 104.3 53) (width 0.25) (layer "B.Cu") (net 12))
 (segment (start 102 57.2) (end 102 62.91) (width 0.25) (layer "B.Cu") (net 12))
 (segment (start 99.0625 57.775) (end 101.075 57.775) (width 0.25) (layer "F.Cu") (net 11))
 (segment (start 116.1 55.6) (end 116.1 53.198964) (width 0.25) (layer "F.Cu") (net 11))
 (segment (start 116.1 53.198964) (end 115.000259 52.099223) (width 0.25) (layer "F.Cu") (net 11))
 (segment (start 101.075 57.775) (end 101.3 58) (width 0.25) (layer "F.Cu") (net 11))
 (segment (start 114.025 57.675) (end 116.1 55.6) (width 0.25) (layer "F.Cu") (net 11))
 (segment (start 113.3625 57.675) (end 114.025 57.675) (width 0.25) (layer "F.Cu") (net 11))
 (via (at 115.000259 52.099223) (size 0.8) (drill 0.4) (layers "F.Cu" "B.Cu") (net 11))
 (via (at 101.3 58) (size 0.8) (drill 0.4) (layers "F.Cu" "B.Cu") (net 11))
 (segment (start 101.3 61.07) (end 94.095 68.275) (width 0.25) (layer "B.Cu") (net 11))
 (segment (start 104.3 52.1) (end 101.325489 55.074511) (width 0.25) (layer "B.Cu") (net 11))
 (segment (start 101.325489 55.074511) (end 101.325489 57.974511) (width 0.25) (layer "B.Cu") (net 11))
 (segment (start 101.3 58) (end 101.3 61.07) (width 0.25) (layer "B.Cu") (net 11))
 (segment (start 114.999482 52.1) (end 104.3 52.1) (width 0.25) (layer "B.Cu") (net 11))
 (segment (start 101.325489 57.974511) (end 101.3 58) (width 0.25) (layer "B.Cu") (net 11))
 (segment (start 115.000259 52.099223) (end 114.999482 52.1) (width 0.25) (layer "B.Cu") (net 11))
 (segment (start 99.0625 59.075) (end 98.445349 59.075) (width 0.25) (layer "F.Cu") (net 15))
 (segment (start 98.445349 59.075) (end 96.5 57.129651) (width 0.25) (layer "F.Cu") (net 15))
 (segment (start 96.5 57.129651) (end 96.5 49) (width 0.25) (layer "F.Cu") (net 15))
 (via (at 96.5 49) (size 0.8) (drill 0.4) (layers "F.Cu" "B.Cu") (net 15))
 (segment (start 96.5 41.5) (end 91.575 36.575) (width 0.25) (layer "B.Cu") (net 15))
 (segment (start 91.575 36.575) (end 91.575 34.325) (width 0.25) (layer "B.Cu") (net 15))
 (segment (start 96.5 49) (end 96.5 41.5) (width 0.25) (layer "B.Cu") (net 15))
 (segment (start 96 50) (end 95.5 50) (width 0.25) (layer "F.Cu") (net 16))
 (segment (start 98.445349 59.725) (end 96 57.279651) (width 0.25) (layer "F.Cu") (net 16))
 (segment (start 99.0625 59.725) (end 98.445349 59.725) (width 0.25) (layer "F.Cu") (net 16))
 (segment (start 96 57.279651) (end 96 50) (width 0.25) (layer "F.Cu") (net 16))
 (via (at 95.5 50) (size 0.8) (drill 0.4) (layers "F.Cu" "B.Cu") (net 16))
 (segment (start 97.174511 40.674511) (end 95.5 39) (width 0.25) (layer "B.Cu") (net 16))
 (segment (start 97.174511 49.279393) (end 97.174511 40.674511) (width 0.25) (layer "B.Cu") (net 16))
 (segment (start 96.453904 50) (end 97.174511 49.279393) (width 0.25) (layer "B.Cu") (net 16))
 (segment (start 94.5 38) (end 95.5 39) (width 0.25) (layer "B.Cu") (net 16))
 (segment (start 94.115 34.325) (end 94.115 37.615) (width 0.25) (layer "B.Cu") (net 16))
 (segment (start 94.115 37.615) (end 94.5 38) (width 0.25) (layer "B.Cu") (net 16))
 (segment (start 95.5 50) (end 96.453904 50) (width 0.25) (layer "B.Cu") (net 16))
 (segment (start 95.5 57.429651) (end 95.5 51) (width 0.25) (layer "F.Cu") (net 17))
 (segment (start 98.445349 60.375) (end 95.5 57.429651) (width 0.25) (layer "F.Cu") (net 17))
 (segment (start 95.5 51) (end 94.5 51) (width 0.25) (layer "F.Cu") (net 17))
 (segment (start 99.0625 60.375) (end 98.445349 60.375) (width 0.25) (layer "F.Cu") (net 17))
 (via (at 94.5 51) (size 0.8) (drill 0.4) (layers "F.Cu" "B.Cu") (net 17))
 (segment (start 97.574031 38.074031) (end 96.655 37.155) (width 0.25) (layer "B.Cu") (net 17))
 (segment (start 94.5 51) (end 96.01891 51) (width 0.25) (layer "B.Cu") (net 17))
 (segment (start 96.655 37.155) (end 96.655 34.325) (width 0.25) (layer "B.Cu") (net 17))
 (segment (start 96.01891 51) (end 97.574031 49.444879) (width 0.25) (layer "B.Cu") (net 17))
 (segment (start 97.574031 49.444879) (end 97.574031 38.074031) (width 0.25) (layer "B.Cu") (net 17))
 (segment (start 111.6745 57.904151) (end 111.6745 50.5) (width 0.25) (layer "F.Cu") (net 9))
 (segment (start 113.3625 58.975) (end 112.745349 58.975) (width 0.25) (layer "F.Cu") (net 9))
 (segment (start 112.745349 58.975) (end 111.6745 57.904151) (width 0.25) (layer "F.Cu") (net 9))
 (via (at 111.6745 50.5) (size 0.8) (drill 0.4) (layers "F.Cu" "B.Cu") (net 9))
 (segment (start 99.195 38.21391) (end 99.195 34.325) (width 0.25) (layer "B.Cu") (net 9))
 (segment (start 111.6745 50.5) (end 111.48109 50.5) (width 0.25) (layer "B.Cu") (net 9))
 (segment (start 111.48109 50.5) (end 99.195 38.21391) (width 0.25) (layer "B.Cu") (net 9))
 (segment (start 112.660355 59.625) (end 111 57.964645) (width 0.25) (layer "F.Cu") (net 8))
 (segment (start 113.3625 59.625) (end 112.660355 59.625) (width 0.25) (layer "F.Cu") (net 8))
 (segment (start 111 57.964645) (end 111 49) (width 0.25) (layer "F.Cu") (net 8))
 (via (at 111 49) (size 0.8) (drill 0.4) (layers "F.Cu" "B.Cu") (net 8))
 (segment (start 109.325489 47.779393) (end 109.325489 45.674511) (width 0.25) (layer "B.Cu") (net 8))
 (segment (start 109.325489 45.674511) (end 101.735 38.084022) (width 0.25) (layer "B.Cu") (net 8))
 (segment (start 101.735 38.084022) (end 101.735 34.325) (width 0.25) (layer "B.Cu") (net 8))
 (segment (start 111 49) (end 110.546096 49) (width 0.25) (layer "B.Cu") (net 8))
 (segment (start 110.546096 49) (end 109.325489 47.779393) (width 0.25) (layer "B.Cu") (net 8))
 (segment (start 110 57.529651) (end 110 47.5) (width 0.25) (layer "F.Cu") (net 7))
 (segment (start 113.3625 60.275) (end 112.745349 60.275) (width 0.25) (layer "F.Cu") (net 7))
 (segment (start 112.745349 60.275) (end 110 57.529651) (width 0.25) (layer "F.Cu") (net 7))
 (via (at 110 47.5) (size 0.8) (drill 0.4) (layers "F.Cu" "B.Cu") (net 7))
 (segment (start 110 43) (end 104.275 37.275) (width 0.25) (layer "B.Cu") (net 7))
 (segment (start 104.275 37.275) (end 104.275 34.325) (width 0.25) (layer "B.Cu") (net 7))
 (segment (start 110 47.5) (end 110 43) (width 0.25) (layer "B.Cu") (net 7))
 (segment (start 101.225 42.275) (end 105 38.5) (width 0.25) (layer "F.Cu") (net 18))
 (segment (start 106.825 38.5) (end 106.9 38.575) (width 0.25) (layer "F.Cu") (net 18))
 (segment (start 105 38.5) (end 106.825 38.5) (width 0.25) (layer "F.Cu") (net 18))
 (segment (start 106.815 34.325) (end 106.815 38.49) (width 0.25) (layer "F.Cu") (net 18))
 (segment (start 100.8125 42.275) (end 101.225 42.275) (width 0.25) (layer "F.Cu") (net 18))
 (segment (start 106.815 38.49) (end 106.9 38.575) (width 0.25) (layer "F.Cu") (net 18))
 (segment (start 106.729408 39.24952) (end 108.87548 39.24952) (width 0.25) (layer "F.Cu") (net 19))
 (segment (start 109.355 34.325) (end 109.355 38.38) (width 0.25) (layer "F.Cu") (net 19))
 (segment (start 109.355 38.38) (end 109.55 38.575) (width 0.25) (layer "F.Cu") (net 19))
 (segment (start 103.053928 42.925) (end 106.729408 39.24952) (width 0.25) (layer "F.Cu") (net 19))
 (segment (start 100.8125 42.925) (end 103.053928 42.925) (width 0.25) (layer "F.Cu") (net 19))
 (segment (start 108.87548 39.24952) (end 109.55 38.575) (width 0.25) (layer "F.Cu") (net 19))
 (segment (start 100.7 49.6) (end 100.8125 49.4875) (width 0.5) (layer "F.Cu") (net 14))
 (segment (start 116.9 36.79) (end 114.435 34.325) (width 0.5) (layer "F.Cu") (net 14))
 (segment (start 113.3625 55.725) (end 113.3625 46.2875) (width 0.5) (layer "F.Cu") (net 14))
 (segment (start 100.8125 49.4875) (end 100.8125 46.5875) (width 0.5) (layer "F.Cu") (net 14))
 (segment (start 113.01 32.9) (end 114.435 34.325) (width 0.25) (layer "F.Cu") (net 14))
 (segment (start 111 32.9) (end 113.01 32.9) (width 0.25) (layer "F.Cu") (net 14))
 (segment (start 110.770489 33.129511) (end 111 32.9) (width 0.25) (layer "F.Cu") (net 14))
 (segment (start 113.475 46.175) (end 116.025 46.175) (width 0.5) (layer "F.Cu") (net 14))
 (segment (start 116.025 46.175) (end 116.9 45.3) (width 0.5) (layer "F.Cu") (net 14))
 (segment (start 114.435 38.41) (end 114.65 38.625) (width 0.5) (layer "F.Cu") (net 14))
 (segment (start 114.435 34.325) (end 114.435 38.41) (width 0.5) (layer "F.Cu") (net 14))
 (segment (start 113.3625 46.2875) (end 113.475 46.175) (width 0.5) (layer "F.Cu") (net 14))
 (segment (start 100.8125 46.825) (end 100.8125 46.5875) (width 0.5) (layer "F.Cu") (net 14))
 (segment (start 99.0625 55.825) (end 99.0625 51.2375) (width 0.5) (layer "F.Cu") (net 14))
 (segment (start 109.55 40.225) (end 110.770489 39.004511) (width 0.25) (layer "F.Cu") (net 14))
 (segment (start 100.8125 46.175) (end 113.475 46.175) (width 0.5) (layer "F.Cu") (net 14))
 (segment (start 99.0625 51.2375) (end 99.6 50.7) (width 0.5) (layer "F.Cu") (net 14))
 (segment (start 106.9 40.225) (end 109.55 40.225) (width 0.25) (layer "F.Cu") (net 14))
 (segment (start 100.8125 46.5875) (end 100.8125 45.525) (width 0.5) (layer "F.Cu") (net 14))
 (segment (start 110.770489 39.004511) (end 110.770489 33.129511) (width 0.25) (layer "F.Cu") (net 14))
 (segment (start 116.9 45.3) (end 116.9 36.79) (width 0.5) (layer "F.Cu") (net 14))
 (via (at 99.6 50.7) (size 0.8) (drill 0.4) (layers "F.Cu" "B.Cu") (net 14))
 (via (at 100.7 49.6) (size 0.8) (drill 0.4) (layers "F.Cu" "B.Cu") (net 14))
 (segment (start 99.6 50.7) (end 100.7 49.6) (width 0.5) (layer "B.Cu") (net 14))
 (segment (start 92.625 57.125) (end 93.3375 57.125) (width 0.25) (layer "F.Cu") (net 24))
 (segment (start 91.5 46.225) (end 91.5 56) (width 0.25) (layer "F.Cu") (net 24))
 (segment (start 91.5 56) (end 92.625 57.125) (width 0.25) (layer "F.Cu") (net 24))
 (segment (start 90.85 44.875) (end 90.5 45.225) (width 0.25) (layer "F.Cu") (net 24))
 (segment (start 90.5 45.225) (end 91.5 46.225) (width 0.25) (layer "F.Cu") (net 24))
 (segment (start 93.9875 44.875) (end 90.85 44.875) (width 0.25) (layer "F.Cu") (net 24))
 (segment (start 93.9875 44.225) (end 91.15 44.225) (width 0.25) (layer "F.Cu") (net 23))
 (segment (start 91.15 44.225) (end 90.5 43.575) (width 0.25) (layer "F.Cu") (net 23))
 (segment (start 95.520349 45.525) (end 107.020349 57.025) (width 0.25) (layer "F.Cu") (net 3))
 (segment (start 93.9875 45.525) (end 95.520349 45.525) (width 0.25) (layer "F.Cu") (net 3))
 (segment (start 107.020349 57.025) (end 107.6375 57.025) (width 0.25) (layer "F.Cu") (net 3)))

